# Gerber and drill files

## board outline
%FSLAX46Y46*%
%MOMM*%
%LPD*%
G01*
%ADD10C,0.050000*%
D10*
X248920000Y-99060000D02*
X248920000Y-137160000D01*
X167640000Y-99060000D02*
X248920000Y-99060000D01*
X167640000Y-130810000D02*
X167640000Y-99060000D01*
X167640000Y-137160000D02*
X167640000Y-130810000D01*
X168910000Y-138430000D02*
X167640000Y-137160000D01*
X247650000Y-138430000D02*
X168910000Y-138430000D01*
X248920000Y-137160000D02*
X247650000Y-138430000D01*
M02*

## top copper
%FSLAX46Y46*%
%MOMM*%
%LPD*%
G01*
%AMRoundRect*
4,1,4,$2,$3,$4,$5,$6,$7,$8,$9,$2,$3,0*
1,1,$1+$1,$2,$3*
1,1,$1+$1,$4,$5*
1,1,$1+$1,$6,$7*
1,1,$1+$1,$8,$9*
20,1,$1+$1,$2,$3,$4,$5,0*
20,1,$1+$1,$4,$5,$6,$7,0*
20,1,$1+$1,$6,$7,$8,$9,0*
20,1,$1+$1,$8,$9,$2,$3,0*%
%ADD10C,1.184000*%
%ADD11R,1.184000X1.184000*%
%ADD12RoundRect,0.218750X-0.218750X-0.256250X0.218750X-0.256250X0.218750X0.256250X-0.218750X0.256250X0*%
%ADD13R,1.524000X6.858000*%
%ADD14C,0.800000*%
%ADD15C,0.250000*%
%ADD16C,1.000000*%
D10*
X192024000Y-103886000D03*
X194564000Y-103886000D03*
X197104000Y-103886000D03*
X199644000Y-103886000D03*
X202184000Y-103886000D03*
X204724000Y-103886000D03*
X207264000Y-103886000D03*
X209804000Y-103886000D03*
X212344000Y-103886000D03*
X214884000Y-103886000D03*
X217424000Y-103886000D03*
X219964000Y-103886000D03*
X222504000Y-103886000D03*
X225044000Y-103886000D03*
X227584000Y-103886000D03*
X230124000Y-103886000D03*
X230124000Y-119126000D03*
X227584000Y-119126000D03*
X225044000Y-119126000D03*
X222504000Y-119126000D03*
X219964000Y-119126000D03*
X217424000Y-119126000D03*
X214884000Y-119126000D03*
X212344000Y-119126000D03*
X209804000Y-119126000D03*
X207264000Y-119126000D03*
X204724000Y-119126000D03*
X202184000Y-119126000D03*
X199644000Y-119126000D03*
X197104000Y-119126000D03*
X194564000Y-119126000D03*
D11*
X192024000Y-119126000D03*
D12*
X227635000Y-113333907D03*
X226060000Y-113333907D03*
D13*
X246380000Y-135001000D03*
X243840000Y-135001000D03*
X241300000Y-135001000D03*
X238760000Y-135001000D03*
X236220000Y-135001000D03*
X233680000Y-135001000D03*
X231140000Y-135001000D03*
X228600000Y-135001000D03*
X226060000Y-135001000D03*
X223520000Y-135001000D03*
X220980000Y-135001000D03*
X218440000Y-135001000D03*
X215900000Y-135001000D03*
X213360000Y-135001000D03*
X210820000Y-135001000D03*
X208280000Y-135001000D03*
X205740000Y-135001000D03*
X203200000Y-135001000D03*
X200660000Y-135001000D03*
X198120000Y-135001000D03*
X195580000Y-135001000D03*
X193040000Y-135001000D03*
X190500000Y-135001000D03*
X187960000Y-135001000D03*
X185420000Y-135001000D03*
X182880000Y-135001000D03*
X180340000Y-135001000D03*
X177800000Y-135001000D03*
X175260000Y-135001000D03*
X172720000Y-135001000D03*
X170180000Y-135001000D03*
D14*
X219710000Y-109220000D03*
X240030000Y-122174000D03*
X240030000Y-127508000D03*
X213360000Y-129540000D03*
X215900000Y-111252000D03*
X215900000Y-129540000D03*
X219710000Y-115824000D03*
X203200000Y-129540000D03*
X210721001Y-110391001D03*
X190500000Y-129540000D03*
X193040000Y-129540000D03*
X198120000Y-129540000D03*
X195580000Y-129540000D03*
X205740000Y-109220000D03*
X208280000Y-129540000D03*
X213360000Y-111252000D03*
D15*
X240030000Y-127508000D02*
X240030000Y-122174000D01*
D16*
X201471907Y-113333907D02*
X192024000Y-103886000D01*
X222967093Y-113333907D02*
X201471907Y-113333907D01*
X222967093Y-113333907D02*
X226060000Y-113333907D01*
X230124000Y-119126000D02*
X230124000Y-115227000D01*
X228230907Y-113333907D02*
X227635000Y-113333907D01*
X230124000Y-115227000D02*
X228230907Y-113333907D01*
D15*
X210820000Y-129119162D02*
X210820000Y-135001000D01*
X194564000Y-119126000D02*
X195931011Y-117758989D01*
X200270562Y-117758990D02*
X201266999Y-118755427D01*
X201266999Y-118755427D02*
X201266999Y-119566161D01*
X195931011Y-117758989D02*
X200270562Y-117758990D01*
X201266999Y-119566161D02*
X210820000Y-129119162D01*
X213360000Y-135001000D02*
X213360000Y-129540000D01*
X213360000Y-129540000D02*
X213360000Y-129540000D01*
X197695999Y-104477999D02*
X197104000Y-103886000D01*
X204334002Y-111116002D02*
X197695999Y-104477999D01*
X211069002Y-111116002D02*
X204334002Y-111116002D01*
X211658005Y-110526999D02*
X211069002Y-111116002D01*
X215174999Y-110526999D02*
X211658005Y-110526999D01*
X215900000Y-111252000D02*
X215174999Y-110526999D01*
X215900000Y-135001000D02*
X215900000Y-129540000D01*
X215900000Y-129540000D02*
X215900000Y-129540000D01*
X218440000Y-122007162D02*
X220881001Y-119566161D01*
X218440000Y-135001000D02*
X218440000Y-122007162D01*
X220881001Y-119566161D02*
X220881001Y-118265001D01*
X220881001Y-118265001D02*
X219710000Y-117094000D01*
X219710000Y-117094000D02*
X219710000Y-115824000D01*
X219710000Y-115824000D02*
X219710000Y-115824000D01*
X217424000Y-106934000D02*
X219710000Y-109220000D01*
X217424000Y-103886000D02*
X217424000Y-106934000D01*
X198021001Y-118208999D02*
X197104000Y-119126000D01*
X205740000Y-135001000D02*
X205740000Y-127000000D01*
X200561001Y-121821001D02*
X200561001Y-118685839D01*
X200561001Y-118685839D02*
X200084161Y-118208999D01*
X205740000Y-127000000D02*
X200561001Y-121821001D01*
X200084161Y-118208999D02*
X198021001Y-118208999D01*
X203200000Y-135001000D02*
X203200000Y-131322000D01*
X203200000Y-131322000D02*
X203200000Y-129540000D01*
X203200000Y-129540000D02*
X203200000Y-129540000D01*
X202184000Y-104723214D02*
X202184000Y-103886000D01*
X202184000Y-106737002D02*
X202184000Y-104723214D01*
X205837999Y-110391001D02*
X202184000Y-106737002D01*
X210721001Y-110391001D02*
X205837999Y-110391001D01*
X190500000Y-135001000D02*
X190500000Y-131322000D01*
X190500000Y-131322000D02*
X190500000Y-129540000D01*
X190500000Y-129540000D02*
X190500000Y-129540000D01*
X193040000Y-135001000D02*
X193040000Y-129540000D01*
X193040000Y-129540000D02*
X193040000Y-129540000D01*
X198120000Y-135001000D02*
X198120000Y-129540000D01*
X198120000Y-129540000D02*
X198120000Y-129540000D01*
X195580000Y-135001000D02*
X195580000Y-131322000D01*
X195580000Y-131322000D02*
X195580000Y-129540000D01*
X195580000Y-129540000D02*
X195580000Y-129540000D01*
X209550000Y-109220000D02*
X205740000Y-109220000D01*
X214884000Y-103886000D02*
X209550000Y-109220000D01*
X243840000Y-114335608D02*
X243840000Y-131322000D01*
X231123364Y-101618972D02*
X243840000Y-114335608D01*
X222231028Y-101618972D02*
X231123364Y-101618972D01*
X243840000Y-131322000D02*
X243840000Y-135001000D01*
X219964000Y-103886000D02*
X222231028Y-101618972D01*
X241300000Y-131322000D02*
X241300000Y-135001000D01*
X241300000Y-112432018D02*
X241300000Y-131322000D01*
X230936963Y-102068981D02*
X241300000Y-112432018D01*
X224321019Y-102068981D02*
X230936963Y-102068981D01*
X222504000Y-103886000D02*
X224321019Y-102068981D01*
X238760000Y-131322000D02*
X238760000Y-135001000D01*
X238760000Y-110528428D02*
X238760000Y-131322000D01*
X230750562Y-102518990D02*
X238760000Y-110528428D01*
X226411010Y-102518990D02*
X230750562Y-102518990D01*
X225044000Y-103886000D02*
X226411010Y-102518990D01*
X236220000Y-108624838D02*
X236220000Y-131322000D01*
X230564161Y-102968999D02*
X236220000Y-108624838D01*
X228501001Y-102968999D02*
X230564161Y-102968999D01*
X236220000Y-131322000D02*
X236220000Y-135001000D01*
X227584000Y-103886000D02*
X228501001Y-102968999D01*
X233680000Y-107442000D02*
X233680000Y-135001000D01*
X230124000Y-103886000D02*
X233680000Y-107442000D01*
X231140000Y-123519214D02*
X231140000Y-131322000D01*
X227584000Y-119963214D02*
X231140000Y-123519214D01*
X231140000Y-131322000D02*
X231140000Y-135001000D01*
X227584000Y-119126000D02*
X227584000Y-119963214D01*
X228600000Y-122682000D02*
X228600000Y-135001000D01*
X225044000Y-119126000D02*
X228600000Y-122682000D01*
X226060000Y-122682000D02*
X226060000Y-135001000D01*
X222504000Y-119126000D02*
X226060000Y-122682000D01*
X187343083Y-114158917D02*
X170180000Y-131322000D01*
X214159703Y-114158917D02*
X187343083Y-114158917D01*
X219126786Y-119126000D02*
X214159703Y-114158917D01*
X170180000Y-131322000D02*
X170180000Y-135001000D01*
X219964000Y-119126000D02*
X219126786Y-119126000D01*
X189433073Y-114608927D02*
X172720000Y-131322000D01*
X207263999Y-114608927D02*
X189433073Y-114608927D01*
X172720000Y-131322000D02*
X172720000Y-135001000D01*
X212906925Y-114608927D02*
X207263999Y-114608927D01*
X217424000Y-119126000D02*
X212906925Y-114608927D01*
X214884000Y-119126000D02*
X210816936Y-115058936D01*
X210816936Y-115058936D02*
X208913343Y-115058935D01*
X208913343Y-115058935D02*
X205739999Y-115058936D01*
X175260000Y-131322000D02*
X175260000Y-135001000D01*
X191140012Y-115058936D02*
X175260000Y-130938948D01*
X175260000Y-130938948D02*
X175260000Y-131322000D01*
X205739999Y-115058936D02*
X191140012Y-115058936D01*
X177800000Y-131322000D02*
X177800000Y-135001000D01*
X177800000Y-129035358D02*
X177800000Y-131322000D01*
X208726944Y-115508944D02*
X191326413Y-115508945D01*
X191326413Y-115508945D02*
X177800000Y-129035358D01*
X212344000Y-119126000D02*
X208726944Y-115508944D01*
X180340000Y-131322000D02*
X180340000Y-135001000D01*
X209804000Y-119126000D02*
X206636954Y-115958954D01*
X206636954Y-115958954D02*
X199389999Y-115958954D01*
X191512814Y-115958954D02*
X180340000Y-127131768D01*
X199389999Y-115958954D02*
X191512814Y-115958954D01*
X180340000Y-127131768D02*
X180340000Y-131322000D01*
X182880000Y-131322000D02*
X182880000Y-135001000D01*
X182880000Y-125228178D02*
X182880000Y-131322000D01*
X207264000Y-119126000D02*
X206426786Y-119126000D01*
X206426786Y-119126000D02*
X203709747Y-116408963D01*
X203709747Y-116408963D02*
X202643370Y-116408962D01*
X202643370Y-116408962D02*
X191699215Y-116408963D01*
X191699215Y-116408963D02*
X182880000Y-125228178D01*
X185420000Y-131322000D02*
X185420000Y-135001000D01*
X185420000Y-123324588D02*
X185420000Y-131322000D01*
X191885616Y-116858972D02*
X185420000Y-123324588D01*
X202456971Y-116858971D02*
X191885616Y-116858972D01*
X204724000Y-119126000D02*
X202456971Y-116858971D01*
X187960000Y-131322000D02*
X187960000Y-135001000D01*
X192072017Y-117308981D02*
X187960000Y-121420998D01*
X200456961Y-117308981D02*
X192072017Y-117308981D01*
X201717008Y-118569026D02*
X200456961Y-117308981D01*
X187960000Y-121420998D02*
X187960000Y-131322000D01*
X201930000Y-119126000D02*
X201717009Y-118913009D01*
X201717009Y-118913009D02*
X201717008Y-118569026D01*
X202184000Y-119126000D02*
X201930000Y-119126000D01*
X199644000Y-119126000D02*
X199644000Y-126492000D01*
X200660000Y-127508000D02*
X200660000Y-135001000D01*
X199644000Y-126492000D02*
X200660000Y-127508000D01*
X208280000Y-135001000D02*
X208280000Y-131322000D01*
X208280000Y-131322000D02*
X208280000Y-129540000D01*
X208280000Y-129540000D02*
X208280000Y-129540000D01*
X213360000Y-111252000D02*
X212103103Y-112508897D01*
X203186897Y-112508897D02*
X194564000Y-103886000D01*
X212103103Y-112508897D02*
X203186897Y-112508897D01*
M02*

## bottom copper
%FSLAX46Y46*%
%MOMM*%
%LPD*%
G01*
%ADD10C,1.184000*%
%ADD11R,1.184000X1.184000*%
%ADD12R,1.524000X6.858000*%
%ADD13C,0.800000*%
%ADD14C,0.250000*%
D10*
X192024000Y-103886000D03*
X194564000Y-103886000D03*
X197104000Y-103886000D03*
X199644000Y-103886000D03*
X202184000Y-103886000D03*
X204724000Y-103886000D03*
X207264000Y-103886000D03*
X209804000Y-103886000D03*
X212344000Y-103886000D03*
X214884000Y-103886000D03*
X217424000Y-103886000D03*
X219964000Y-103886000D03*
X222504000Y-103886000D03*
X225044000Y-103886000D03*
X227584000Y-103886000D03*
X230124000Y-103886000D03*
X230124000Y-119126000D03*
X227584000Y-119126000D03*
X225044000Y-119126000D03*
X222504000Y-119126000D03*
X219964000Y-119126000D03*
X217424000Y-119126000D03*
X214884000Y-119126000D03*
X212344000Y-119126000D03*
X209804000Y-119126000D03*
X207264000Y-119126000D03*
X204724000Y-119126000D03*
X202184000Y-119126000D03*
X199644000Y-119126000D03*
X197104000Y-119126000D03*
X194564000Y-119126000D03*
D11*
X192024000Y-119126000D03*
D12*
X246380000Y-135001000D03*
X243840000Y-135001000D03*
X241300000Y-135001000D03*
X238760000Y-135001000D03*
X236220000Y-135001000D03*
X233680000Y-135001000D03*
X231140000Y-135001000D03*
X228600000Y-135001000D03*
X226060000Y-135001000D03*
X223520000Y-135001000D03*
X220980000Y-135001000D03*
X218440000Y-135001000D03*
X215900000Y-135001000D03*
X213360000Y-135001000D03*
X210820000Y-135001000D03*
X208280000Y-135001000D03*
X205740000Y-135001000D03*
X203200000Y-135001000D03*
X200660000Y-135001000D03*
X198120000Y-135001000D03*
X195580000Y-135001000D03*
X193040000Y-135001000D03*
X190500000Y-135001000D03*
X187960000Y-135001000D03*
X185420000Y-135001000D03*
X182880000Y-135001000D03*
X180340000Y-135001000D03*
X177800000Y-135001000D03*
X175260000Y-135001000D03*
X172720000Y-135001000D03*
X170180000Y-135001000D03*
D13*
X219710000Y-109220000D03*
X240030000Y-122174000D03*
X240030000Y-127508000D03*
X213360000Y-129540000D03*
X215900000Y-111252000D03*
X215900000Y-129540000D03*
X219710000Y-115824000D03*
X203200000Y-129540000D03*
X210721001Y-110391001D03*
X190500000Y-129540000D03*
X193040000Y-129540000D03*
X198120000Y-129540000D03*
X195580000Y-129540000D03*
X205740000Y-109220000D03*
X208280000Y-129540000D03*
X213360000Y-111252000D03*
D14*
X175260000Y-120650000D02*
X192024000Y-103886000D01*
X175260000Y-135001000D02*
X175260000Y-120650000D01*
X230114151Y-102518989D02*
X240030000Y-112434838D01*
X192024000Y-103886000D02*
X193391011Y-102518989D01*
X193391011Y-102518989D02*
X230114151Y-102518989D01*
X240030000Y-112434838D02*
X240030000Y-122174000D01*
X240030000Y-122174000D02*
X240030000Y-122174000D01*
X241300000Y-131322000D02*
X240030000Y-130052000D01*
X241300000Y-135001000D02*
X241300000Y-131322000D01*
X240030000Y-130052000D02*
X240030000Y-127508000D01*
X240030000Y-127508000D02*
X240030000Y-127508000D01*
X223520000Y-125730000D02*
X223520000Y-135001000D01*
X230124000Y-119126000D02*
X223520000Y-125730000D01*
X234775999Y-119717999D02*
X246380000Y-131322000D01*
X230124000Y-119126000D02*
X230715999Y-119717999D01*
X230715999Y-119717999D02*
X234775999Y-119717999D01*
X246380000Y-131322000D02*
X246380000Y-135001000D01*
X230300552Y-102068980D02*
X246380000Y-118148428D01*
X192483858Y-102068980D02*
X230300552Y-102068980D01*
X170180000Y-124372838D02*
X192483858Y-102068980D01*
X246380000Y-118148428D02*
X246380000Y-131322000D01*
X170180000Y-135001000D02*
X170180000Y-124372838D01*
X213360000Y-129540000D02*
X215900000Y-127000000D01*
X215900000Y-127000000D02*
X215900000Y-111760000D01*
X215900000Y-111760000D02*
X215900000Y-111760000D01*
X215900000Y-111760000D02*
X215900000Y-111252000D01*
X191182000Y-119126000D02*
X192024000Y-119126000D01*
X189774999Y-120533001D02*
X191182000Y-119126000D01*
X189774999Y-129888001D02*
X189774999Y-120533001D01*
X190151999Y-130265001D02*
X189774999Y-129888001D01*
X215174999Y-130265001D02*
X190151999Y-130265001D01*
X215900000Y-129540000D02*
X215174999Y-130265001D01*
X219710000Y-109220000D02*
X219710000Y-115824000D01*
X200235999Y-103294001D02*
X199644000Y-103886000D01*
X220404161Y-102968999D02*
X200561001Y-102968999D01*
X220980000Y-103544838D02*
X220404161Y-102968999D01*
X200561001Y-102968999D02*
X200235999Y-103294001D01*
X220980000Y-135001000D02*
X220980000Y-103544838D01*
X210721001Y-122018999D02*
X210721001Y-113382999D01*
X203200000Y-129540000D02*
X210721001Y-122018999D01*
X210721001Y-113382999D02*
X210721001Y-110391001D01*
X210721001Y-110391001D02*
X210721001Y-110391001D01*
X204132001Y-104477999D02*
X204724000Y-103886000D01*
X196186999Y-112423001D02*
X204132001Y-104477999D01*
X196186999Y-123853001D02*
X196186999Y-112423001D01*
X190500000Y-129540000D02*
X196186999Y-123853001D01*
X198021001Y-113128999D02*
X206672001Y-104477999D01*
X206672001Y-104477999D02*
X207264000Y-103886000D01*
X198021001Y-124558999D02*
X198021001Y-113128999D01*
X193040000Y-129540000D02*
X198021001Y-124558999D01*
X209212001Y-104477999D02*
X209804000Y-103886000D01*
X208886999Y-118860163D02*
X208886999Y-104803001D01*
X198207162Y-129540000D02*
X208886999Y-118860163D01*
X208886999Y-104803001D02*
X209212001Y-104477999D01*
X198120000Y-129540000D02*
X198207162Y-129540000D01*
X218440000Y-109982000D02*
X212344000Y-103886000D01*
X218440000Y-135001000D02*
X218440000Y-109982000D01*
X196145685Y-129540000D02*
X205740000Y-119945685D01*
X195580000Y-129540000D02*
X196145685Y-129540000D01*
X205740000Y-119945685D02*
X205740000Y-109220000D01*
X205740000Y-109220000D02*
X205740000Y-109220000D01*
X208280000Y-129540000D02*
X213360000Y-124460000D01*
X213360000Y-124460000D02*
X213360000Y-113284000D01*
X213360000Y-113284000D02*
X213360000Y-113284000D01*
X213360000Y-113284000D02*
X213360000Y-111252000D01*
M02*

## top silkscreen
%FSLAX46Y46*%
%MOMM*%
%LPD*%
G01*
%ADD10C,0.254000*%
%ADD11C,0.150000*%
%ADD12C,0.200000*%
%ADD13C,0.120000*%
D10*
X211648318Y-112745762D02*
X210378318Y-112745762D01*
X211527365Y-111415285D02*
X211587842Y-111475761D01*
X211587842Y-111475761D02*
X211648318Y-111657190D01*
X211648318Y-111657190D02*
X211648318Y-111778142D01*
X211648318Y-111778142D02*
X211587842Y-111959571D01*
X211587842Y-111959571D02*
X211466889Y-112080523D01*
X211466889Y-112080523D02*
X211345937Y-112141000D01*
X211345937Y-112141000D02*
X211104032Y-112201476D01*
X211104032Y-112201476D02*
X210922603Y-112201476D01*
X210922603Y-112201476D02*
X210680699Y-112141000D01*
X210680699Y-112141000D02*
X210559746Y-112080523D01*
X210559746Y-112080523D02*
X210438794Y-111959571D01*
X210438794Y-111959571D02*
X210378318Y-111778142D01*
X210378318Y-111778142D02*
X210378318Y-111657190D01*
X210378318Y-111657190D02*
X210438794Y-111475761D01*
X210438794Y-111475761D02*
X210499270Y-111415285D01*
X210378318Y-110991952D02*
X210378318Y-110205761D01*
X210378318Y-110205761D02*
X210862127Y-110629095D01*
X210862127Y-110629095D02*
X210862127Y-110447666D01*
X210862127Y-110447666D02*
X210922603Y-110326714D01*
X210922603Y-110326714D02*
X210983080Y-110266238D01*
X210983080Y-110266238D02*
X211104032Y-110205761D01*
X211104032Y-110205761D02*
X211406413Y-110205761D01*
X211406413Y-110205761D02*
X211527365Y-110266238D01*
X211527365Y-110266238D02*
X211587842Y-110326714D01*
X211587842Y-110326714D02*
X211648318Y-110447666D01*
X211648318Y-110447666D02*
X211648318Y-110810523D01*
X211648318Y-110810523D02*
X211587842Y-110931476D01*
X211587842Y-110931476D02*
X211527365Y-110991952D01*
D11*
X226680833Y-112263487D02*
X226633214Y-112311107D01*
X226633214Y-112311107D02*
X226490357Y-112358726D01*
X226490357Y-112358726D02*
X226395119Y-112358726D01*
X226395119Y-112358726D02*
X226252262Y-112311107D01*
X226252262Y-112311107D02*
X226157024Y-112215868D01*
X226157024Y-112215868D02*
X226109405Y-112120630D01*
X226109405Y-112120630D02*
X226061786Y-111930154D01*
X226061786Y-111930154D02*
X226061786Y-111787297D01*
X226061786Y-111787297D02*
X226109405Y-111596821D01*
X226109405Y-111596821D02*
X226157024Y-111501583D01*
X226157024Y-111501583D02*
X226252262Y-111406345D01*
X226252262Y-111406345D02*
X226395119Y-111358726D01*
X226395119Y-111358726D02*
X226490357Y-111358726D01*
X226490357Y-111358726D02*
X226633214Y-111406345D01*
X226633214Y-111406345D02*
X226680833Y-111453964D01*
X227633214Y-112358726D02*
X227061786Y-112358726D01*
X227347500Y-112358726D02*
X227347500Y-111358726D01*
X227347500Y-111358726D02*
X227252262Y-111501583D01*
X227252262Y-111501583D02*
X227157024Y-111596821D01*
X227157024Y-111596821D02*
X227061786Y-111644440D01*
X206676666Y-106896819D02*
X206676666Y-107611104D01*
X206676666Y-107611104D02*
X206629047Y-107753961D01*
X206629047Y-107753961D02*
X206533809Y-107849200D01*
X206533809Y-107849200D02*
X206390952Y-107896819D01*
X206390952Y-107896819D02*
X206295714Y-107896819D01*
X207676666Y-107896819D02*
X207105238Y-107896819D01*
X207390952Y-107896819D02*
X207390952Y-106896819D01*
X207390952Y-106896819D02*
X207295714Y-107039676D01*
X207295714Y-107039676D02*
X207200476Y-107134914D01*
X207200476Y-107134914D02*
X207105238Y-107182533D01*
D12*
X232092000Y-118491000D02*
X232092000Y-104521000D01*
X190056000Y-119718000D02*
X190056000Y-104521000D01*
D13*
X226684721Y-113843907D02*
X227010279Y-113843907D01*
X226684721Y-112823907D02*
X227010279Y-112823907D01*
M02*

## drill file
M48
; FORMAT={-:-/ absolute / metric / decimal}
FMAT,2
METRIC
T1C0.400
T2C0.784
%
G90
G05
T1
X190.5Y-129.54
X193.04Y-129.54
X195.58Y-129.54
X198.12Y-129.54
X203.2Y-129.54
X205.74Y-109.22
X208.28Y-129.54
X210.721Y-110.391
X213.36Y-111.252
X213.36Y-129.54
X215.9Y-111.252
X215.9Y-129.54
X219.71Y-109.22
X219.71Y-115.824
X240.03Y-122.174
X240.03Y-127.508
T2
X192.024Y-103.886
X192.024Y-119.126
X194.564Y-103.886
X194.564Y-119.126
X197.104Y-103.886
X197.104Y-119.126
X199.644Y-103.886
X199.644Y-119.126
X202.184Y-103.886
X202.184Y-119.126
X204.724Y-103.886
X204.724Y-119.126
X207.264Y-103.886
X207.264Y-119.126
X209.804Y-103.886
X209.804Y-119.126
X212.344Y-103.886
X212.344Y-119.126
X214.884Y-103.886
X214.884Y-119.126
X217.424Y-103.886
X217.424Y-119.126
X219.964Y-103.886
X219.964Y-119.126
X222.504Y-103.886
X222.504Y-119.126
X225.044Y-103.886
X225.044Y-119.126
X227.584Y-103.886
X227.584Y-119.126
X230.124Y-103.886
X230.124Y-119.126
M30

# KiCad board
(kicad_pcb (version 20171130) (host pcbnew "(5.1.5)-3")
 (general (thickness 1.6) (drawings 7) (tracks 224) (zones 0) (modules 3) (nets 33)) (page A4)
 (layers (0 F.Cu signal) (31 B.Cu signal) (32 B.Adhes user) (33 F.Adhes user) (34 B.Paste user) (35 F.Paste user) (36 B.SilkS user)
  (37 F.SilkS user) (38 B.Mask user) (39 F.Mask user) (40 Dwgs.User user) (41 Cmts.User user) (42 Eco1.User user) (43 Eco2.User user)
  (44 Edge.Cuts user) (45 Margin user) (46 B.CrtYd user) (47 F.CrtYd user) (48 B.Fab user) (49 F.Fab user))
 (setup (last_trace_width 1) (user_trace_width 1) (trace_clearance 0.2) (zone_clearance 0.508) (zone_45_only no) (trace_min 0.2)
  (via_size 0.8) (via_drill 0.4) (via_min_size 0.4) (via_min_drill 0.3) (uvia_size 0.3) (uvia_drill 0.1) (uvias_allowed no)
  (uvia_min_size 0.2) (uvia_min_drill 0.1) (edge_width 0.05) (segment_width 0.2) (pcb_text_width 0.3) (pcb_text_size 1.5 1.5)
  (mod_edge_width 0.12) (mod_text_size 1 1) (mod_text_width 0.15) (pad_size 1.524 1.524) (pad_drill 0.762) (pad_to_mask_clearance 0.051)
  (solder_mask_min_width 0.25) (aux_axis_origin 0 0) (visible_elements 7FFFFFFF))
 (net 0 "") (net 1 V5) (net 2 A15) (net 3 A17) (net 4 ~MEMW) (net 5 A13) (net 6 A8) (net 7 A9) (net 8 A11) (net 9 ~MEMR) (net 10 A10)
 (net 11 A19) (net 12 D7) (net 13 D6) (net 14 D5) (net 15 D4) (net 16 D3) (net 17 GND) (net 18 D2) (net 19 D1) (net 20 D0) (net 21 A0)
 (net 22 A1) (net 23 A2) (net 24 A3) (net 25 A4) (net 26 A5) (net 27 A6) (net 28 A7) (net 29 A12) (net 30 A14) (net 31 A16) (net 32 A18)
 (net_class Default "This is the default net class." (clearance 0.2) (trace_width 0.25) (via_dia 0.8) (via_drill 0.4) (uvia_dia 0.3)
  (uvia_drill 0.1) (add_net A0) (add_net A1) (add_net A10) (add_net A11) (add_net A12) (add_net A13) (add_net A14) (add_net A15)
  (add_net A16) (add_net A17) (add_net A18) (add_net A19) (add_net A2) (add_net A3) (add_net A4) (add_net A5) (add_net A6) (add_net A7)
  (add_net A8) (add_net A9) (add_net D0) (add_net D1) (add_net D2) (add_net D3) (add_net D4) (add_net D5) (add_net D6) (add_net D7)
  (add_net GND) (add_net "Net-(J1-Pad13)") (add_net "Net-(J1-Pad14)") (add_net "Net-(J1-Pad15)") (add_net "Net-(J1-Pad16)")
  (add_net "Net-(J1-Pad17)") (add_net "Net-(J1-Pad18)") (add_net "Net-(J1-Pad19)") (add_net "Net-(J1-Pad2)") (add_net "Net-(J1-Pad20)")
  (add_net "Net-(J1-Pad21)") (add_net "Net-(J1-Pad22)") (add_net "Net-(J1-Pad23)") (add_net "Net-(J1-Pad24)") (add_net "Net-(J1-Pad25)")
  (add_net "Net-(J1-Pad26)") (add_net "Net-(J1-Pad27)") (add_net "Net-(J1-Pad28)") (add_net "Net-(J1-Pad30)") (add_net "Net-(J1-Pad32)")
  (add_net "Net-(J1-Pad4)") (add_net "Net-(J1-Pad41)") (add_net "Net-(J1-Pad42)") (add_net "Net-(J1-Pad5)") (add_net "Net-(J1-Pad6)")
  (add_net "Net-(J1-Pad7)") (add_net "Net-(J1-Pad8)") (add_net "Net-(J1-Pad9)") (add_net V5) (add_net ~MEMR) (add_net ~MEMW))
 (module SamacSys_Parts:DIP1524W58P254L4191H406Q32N (layer F.Cu) (at 211.074 111.506 90)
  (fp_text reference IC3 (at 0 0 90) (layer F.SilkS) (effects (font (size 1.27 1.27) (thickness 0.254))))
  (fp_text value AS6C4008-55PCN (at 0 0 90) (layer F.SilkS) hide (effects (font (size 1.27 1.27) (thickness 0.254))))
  (fp_line (start -6.985 21.018) (end 6.985 21.018) (layer F.SilkS) (width 0.2))
  (fp_line (start -8.212 -21.018) (end 6.985 -21.018) (layer F.SilkS) (width 0.2))
  (pad 32 thru_hole circle (at 7.62 -19.05 90) (size 1.184 1.184) (drill 0.784) (layers *.Cu *.Mask) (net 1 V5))
  (pad 31 thru_hole circle (at 7.62 -16.51 90) (size 1.184 1.184) (drill 0.784) (layers *.Cu *.Mask) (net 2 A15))
  (pad 30 thru_hole circle (at 7.62 -13.97 90) (size 1.184 1.184) (drill 0.784) (layers *.Cu *.Mask) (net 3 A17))
  (pad 29 thru_hole circle (at 7.62 -11.43 90) (size 1.184 1.184) (drill 0.784) (layers *.Cu *.Mask) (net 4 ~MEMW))
  (pad 28 thru_hole circle (at 7.62 -8.89 90) (size 1.184 1.184) (drill 0.784) (layers *.Cu *.Mask) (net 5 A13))
  (pad 27 thru_hole circle (at 7.62 -6.35 90) (size 1.184 1.184) (drill 0.784) (layers *.Cu *.Mask) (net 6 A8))
  (pad 26 thru_hole circle (at 7.62 -3.81 90) (size 1.184 1.184) (drill 0.784) (layers *.Cu *.Mask) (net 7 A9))
  (pad 25 thru_hole circle (at 7.62 -1.27 90) (size 1.184 1.184) (drill 0.784) (layers *.Cu *.Mask) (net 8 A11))
  (pad 24 thru_hole circle (at 7.62 1.27 90) (size 1.184 1.184) (drill 0.784) (layers *.Cu *.Mask) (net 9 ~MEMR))
  (pad 23 thru_hole circle (at 7.62 3.81 90) (size 1.184 1.184) (drill 0.784) (layers *.Cu *.Mask) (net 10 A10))
  (pad 22 thru_hole circle (at 7.62 6.35 90) (size 1.184 1.184) (drill 0.784) (layers *.Cu *.Mask) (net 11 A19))
  (pad 21 thru_hole circle (at 7.62 8.89 90) (size 1.184 1.184) (drill 0.784) (layers *.Cu *.Mask) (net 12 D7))
  (pad 20 thru_hole circle (at 7.62 11.43 90) (size 1.184 1.184) (drill 0.784) (layers *.Cu *.Mask) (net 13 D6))
  (pad 19 thru_hole circle (at 7.62 13.97 90) (size 1.184 1.184) (drill 0.784) (layers *.Cu *.Mask) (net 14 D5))
  (pad 18 thru_hole circle (at 7.62 16.51 90) (size 1.184 1.184) (drill 0.784) (layers *.Cu *.Mask) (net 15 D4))
  (pad 17 thru_hole circle (at 7.62 19.05 90) (size 1.184 1.184) (drill 0.784) (layers *.Cu *.Mask) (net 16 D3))
  (pad 16 thru_hole circle (at -7.62 19.05 90) (size 1.184 1.184) (drill 0.784) (layers *.Cu *.Mask) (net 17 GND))
  (pad 15 thru_hole circle (at -7.62 16.51 90) (size 1.184 1.184) (drill 0.784) (layers *.Cu *.Mask) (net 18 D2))
  (pad 14 thru_hole circle (at -7.62 13.97 90) (size 1.184 1.184) (drill 0.784) (layers *.Cu *.Mask) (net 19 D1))
  (pad 13 thru_hole circle (at -7.62 11.43 90) (size 1.184 1.184) (drill 0.784) (layers *.Cu *.Mask) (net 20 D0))
  (pad 12 thru_hole circle (at -7.62 8.89 90) (size 1.184 1.184) (drill 0.784) (layers *.Cu *.Mask) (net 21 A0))
  (pad 11 thru_hole circle (at -7.62 6.35 90) (size 1.184 1.184) (drill 0.784) (layers *.Cu *.Mask) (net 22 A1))
  (pad 10 thru_hole circle (at -7.62 3.81 90) (size 1.184 1.184) (drill 0.784) (layers *.Cu *.Mask) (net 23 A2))
  (pad 9 thru_hole circle (at -7.62 1.27 90) (size 1.184 1.184) (drill 0.784) (layers *.Cu *.Mask) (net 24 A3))
  (pad 8 thru_hole circle (at -7.62 -1.27 90) (size 1.184 1.184) (drill 0.784) (layers *.Cu *.Mask) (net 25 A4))
  (pad 7 thru_hole circle (at -7.62 -3.81 90) (size 1.184 1.184) (drill 0.784) (layers *.Cu *.Mask) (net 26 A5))
  (pad 6 thru_hole circle (at -7.62 -6.35 90) (size 1.184 1.184) (drill 0.784) (layers *.Cu *.Mask) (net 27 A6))
  (pad 5 thru_hole circle (at -7.62 -8.89 90) (size 1.184 1.184) (drill 0.784) (layers *.Cu *.Mask) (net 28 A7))
  (pad 4 thru_hole circle (at -7.62 -11.43 90) (size 1.184 1.184) (drill 0.784) (layers *.Cu *.Mask) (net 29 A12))
  (pad 3 thru_hole circle (at -7.62 -13.97 90) (size 1.184 1.184) (drill 0.784) (layers *.Cu *.Mask) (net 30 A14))
  (pad 2 thru_hole circle (at -7.62 -16.51 90) (size 1.184 1.184) (drill 0.784) (layers *.Cu *.Mask) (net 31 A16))
  (pad 1 thru_hole rect (at -7.62 -19.05 90) (size 1.184 1.184) (drill 0.784) (layers *.Cu *.Mask) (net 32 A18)))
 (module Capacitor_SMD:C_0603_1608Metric (layer F.Cu) (at 226.8475 113.333907)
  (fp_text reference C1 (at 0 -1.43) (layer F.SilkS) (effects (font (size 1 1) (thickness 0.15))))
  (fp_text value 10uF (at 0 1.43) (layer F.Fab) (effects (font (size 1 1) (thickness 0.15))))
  (fp_line (start -0.162779 0.51) (end 0.162779 0.51) (layer F.SilkS) (width 0.12))
  (fp_line (start -0.162779 -0.51) (end 0.162779 -0.51) (layer F.SilkS) (width 0.12))
  (pad 2 smd roundrect (at 0.7875 0) (size 0.875 0.95) (layers F.Cu F.Paste F.Mask) (roundrect_rratio 0.25) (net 17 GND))
  (pad 1 smd roundrect (at -0.7875 0) (size 0.875 0.95) (layers F.Cu F.Paste F.Mask) (roundrect_rratio 0.25) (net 1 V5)))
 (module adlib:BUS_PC (layer F.Cu) (at 208.28 134.62)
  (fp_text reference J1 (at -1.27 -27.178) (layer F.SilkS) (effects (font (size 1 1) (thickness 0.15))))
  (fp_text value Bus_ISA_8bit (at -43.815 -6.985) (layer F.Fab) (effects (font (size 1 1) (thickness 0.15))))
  (pad 1 connect rect (at 38.1 0.381) (size 1.524 6.858) (layers B.Cu B.Mask) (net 17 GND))
  (pad 2 connect rect (at 35.56 0.381) (size 1.524 6.858) (layers B.Cu B.Mask))
  (pad 3 connect rect (at 33.02 0.381) (size 1.524 6.858) (layers B.Cu B.Mask) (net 1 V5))
  (pad 4 connect rect (at 30.48 0.381) (size 1.524 6.858) (layers B.Cu B.Mask))
  (pad 5 connect rect (at 27.94 0.381) (size 1.524 6.858) (layers B.Cu B.Mask))
  (pad 6 connect rect (at 25.4 0.381) (size 1.524 6.858) (layers B.Cu B.Mask))
  (pad 7 connect rect (at 22.86 0.381) (size 1.524 6.858) (layers B.Cu B.Mask))
  (pad 8 connect rect (at 20.32 0.381) (size 1.524 6.858) (layers B.Cu B.Mask))
  (pad 9 connect rect (at 17.78 0.381) (size 1.524 6.858) (layers B.Cu B.Mask))
  (pad 10 connect rect (at 15.24 0.381) (size 1.524 6.858) (layers B.Cu B.Mask) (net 17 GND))
  (pad 11 connect rect (at 12.7 0.381) (size 1.524 6.858) (layers B.Cu B.Mask) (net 4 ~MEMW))
  (pad 12 connect rect (at 10.16 0.381) (size 1.524 6.858) (layers B.Cu B.Mask) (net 9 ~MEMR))
  (pad 13 connect rect (at 7.62 0.381) (size 1.524 6.858) (layers B.Cu B.Mask))
  (pad 14 connect rect (at 5.08 0.381) (size 1.524 6.858) (layers B.Cu B.Mask))
  (pad 15 connect rect (at 2.54 0.381) (size 1.524 6.858) (layers B.Cu B.Mask))
  (pad 16 connect rect (at 0 0.381) (size 1.524 6.858) (layers B.Cu B.Mask))
  (pad 17 connect rect (at -2.54 0.381) (size 1.524 6.858) (layers B.Cu B.Mask))
  (pad 18 connect rect (at -5.08 0.381) (size 1.524 6.858) (layers B.Cu B.Mask))
  (pad 19 connect rect (at -7.62 0.381) (size 1.524 6.858) (layers B.Cu B.Mask))
  (pad 20 connect rect (at -10.16 0.381) (size 1.524 6.858) (layers B.Cu B.Mask))
  (pad 21 connect rect (at -12.7 0.381) (size 1.524 6.858) (layers B.Cu B.Mask))
  (pad 22 connect rect (at -15.24 0.381) (size 1.524 6.858) (layers B.Cu B.Mask))
  (pad 23 connect rect (at -17.78 0.381) (size 1.524 6.858) (layers B.Cu B.Mask))
  (pad 24 connect rect (at -20.32 0.381) (size 1.524 6.858) (layers B.Cu B.Mask))
  (pad 25 connect rect (at -22.86 0.381) (size 1.524 6.858) (layers B.Cu B.Mask))
  (pad 26 connect rect (at -25.4 0.381) (size 1.524 6.858) (layers B.Cu B.Mask))
  (pad 27 connect rect (at -27.94 0.381) (size 1.524 6.858) (layers B.Cu B.Mask))
  (pad 28 connect rect (at -30.48 0.381) (size 1.524 6.858) (layers B.Cu B.Mask))
  (pad 29 connect rect (at -33.02 0.381) (size 1.524 6.858) (layers B.Cu B.Mask) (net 1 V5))
  (pad 30 connect rect (at -35.56 0.381) (size 1.524 6.858) (layers B.Cu B.Mask))
  (pad 31 connect rect (at -38.1 0.381) (size 1.524 6.858) (layers B.Cu B.Mask) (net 17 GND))
  (pad 32 connect rect (at 38.1 0.381) (size 1.524 6.858) (layers F.Cu F.Mask))
  (pad 33 connect rect (at 35.56 0.381) (size 1.524 6.858) (layers F.Cu F.Mask) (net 12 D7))
  (pad 34 connect rect (at 33.02 0.381) (size 1.524 6.858) (layers F.Cu F.Mask) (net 13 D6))
  (pad 35 connect rect (at 30.48 0.381) (size 1.524 6.858) (layers F.Cu F.Mask) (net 14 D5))
  (pad 36 connect rect (at 27.94 0.381) (size 1.524 6.858) (layers F.Cu F.Mask) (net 15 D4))
  (pad 37 connect rect (at 25.4 0.381) (size 1.524 6.858) (layers F.Cu F.Mask) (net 16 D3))
  (pad 38 connect rect (at 22.86 0.381) (size 1.524 6.858) (layers F.Cu F.Mask) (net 18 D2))
  (pad 39 connect rect (at 20.32 0.381) (size 1.524 6.858) (layers F.Cu F.Mask) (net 19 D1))
  (pad 40 connect rect (at 17.78 0.381) (size 1.524 6.858) (layers F.Cu F.Mask) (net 20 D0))
  (pad 41 connect rect (at 15.24 0.381) (size 1.524 6.858) (layers F.Cu F.Mask))
  (pad 42 connect rect (at 12.7 0.381) (size 1.524 6.858) (layers F.Cu F.Mask))
  (pad 43 connect rect (at 10.16 0.381) (size 1.524 6.858) (layers F.Cu F.Mask) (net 11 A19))
  (pad 44 connect rect (at 7.62 0.381) (size 1.524 6.858) (layers F.Cu F.Mask) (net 32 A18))
  (pad 45 connect rect (at 5.08 0.381) (size 1.524 6.858) (layers F.Cu F.Mask) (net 3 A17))
  (pad 46 connect rect (at 2.54 0.381) (size 1.524 6.858) (layers F.Cu F.Mask) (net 31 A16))
  (pad 47 connect rect (at 0 0.381) (size 1.524 6.858) (layers F.Cu F.Mask) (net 2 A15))
  (pad 48 connect rect (at -2.54 0.381) (size 1.524 6.858) (layers F.Cu F.Mask) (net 30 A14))
  (pad 49 connect rect (at -5.08 0.381) (size 1.524 6.858) (layers F.Cu F.Mask) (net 5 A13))
  (pad 50 connect rect (at -7.62 0.381) (size 1.524 6.858) (layers F.Cu F.Mask) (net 29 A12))
  (pad 51 connect rect (at -10.16 0.381) (size 1.524 6.858) (layers F.Cu F.Mask) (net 8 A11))
  (pad 52 connect rect (at -12.7 0.381) (size 1.524 6.858) (layers F.Cu F.Mask) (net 10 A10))
  (pad 53 connect rect (at -15.24 0.381) (size 1.524 6.858) (layers F.Cu F.Mask) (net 7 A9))
  (pad 54 connect rect (at -17.78 0.381) (size 1.524 6.858) (layers F.Cu F.Mask) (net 6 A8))
  (pad 55 connect rect (at -20.32 0.381) (size 1.524 6.858) (layers F.Cu F.Mask) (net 28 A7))
  (pad 56 connect rect (at -22.86 0.381) (size 1.524 6.858) (layers F.Cu F.Mask) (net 27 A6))
  (pad 57 connect rect (at -25.4 0.381) (size 1.524 6.858) (layers F.Cu F.Mask) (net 26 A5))
  (pad 58 connect rect (at -27.94 0.381) (size 1.524 6.858) (layers F.Cu F.Mask) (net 25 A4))
  (pad 59 connect rect (at -30.48 0.381) (size 1.524 6.858) (layers F.Cu F.Mask) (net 24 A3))
  (pad 60 connect rect (at -33.02 0.381) (size 1.524 6.858) (layers F.Cu F.Mask) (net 23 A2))
  (pad 61 connect rect (at -35.56 0.381) (size 1.524 6.858) (layers F.Cu F.Mask) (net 22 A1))
  (pad 62 connect rect (at -38.1 0.381) (size 1.524 6.858) (layers F.Cu F.Mask) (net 21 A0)))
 (gr_line (start 248.92 99.06) (end 248.92 137.16) (layer Edge.Cuts) (width 0.05))
 (gr_line (start 167.64 99.06) (end 248.92 99.06) (layer Edge.Cuts) (width 0.05))
 (gr_line (start 167.64 130.81) (end 167.64 99.06) (layer Edge.Cuts) (width 0.05))
 (gr_line (start 167.64 137.16) (end 167.64 130.81) (layer Edge.Cuts) (width 0.05))
 (gr_line (start 168.91 138.43) (end 167.64 137.16) (layer Edge.Cuts) (width 0.05))
 (gr_line (start 247.65 138.43) (end 168.91 138.43) (layer Edge.Cuts) (width 0.05))
 (gr_line (start 248.92 137.16) (end 247.65 138.43) (layer Edge.Cuts) (width 0.05))
 (via (at 219.71 109.22) (size 0.8) (drill 0.4) (layers F.Cu B.Cu) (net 11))
 (segment (start 175.26 120.65) (end 192.024 103.886) (width 0.25) (layer B.Cu) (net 1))
 (segment (start 175.26 135.001) (end 175.26 120.65) (width 0.25) (layer B.Cu) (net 1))
 (segment (start 230.114151 102.518989) (end 240.03 112.434838) (width 0.25) (layer B.Cu) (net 1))
 (segment (start 192.024 103.886) (end 193.391011 102.518989) (width 0.25) (layer B.Cu) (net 1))
 (segment (start 193.391011 102.518989) (end 230.114151 102.518989) (width 0.25) (layer B.Cu) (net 1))
 (segment (start 240.03 112.434838) (end 240.03 122.174) (width 0.25) (layer B.Cu) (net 1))
 (segment (start 240.03 122.174) (end 240.03 122.174) (width 0.25) (layer B.Cu) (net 1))
 (via (at 240.03 122.174) (size 0.8) (drill 0.4) (layers F.Cu B.Cu) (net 1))
 (segment (start 241.3 131.322) (end 240.03 130.052) (width 0.25) (layer B.Cu) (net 1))
 (segment (start 241.3 135.001) (end 241.3 131.322) (width 0.25) (layer B.Cu) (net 1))
 (segment (start 240.03 130.052) (end 240.03 127.508) (width 0.25) (layer B.Cu) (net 1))
 (segment (start 240.03 127.508) (end 240.03 127.508) (width 0.25) (layer B.Cu) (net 1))
 (via (at 240.03 127.508) (size 0.8) (drill 0.4) (layers F.Cu B.Cu) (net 1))
 (segment (start 240.03 127.508) (end 240.03 122.174) (width 0.25) (layer F.Cu) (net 1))
 (segment (start 201.471907 113.333907) (end 192.024 103.886) (width 1) (layer F.Cu) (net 1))
 (segment (start 222.967093 113.333907) (end 201.471907 113.333907) (width 1) (layer F.Cu) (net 1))
 (segment (start 222.967093 113.333907) (end 226.06 113.333907) (width 1) (layer F.Cu) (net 1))
 (segment (start 223.52 125.73) (end 223.52 135.001) (width 0.25) (layer B.Cu) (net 17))
 (segment (start 230.124 119.126) (end 223.52 125.73) (width 0.25) (layer B.Cu) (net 17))
 (segment (start 234.775999 119.717999) (end 246.38 131.322) (width 0.25) (layer B.Cu) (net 17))
 (segment (start 230.124 119.126) (end 230.715999 119.717999) (width 0.25) (layer B.Cu) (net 17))
 (segment (start 230.715999 119.717999) (end 234.775999 119.717999) (width 0.25) (layer B.Cu) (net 17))
 (segment (start 246.38 131.322) (end 246.38 135.001) (width 0.25) (layer B.Cu) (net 17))
 (segment (start 230.300552 102.06898) (end 246.38 118.148428) (width 0.25) (layer B.Cu) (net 17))
 (segment (start 192.483858 102.06898) (end 230.300552 102.06898) (width 0.25) (layer B.Cu) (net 17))
 (segment (start 170.18 124.372838) (end 192.483858 102.06898) (width 0.25) (layer B.Cu) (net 17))
 (segment (start 246.38 118.148428) (end 246.38 131.322) (width 0.25) (layer B.Cu) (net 17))
 (segment (start 170.18 135.001) (end 170.18 124.372838) (width 0.25) (layer B.Cu) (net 17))
 (segment (start 230.124 119.126) (end 230.124 115.227) (width 1) (layer F.Cu) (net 17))
 (segment (start 228.230907 113.333907) (end 227.635 113.333907) (width 1) (layer F.Cu) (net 17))
 (segment (start 230.124 115.227) (end 228.230907 113.333907) (width 1) (layer F.Cu) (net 17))
 (segment (start 210.82 129.119162) (end 210.82 135.001) (width 0.25) (layer F.Cu) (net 31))
 (segment (start 194.564 119.126) (end 195.931011 117.758989) (width 0.25) (layer F.Cu) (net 31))
 (segment (start 200.270562 117.75899) (end 201.266999 118.755427) (width 0.25) (layer F.Cu) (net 31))
 (segment (start 201.266999 118.755427) (end 201.266999 119.566161) (width 0.25) (layer F.Cu) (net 31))
 (segment (start 195.931011 117.758989) (end 200.270562 117.75899) (width 0.25) (layer F.Cu) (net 31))
 (segment (start 201.266999 119.566161) (end 210.82 129.119162) (width 0.25) (layer F.Cu) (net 31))
 (segment (start 213.36 135.001) (end 213.36 129.54) (width 0.25) (layer F.Cu) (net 3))
 (segment (start 213.36 129.54) (end 213.36 129.54) (width 0.25) (layer F.Cu) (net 3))
 (via (at 213.36 129.54) (size 0.8) (drill 0.4) (layers F.Cu B.Cu) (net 3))
 (segment (start 213.36 129.54) (end 215.9 127) (width 0.25) (layer B.Cu) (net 3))
 (segment (start 215.9 127) (end 215.9 111.76) (width 0.25) (layer B.Cu) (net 3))
 (segment (start 215.9 111.76) (end 215.9 111.76) (width 0.25) (layer B.Cu) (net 3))
 (via (at 215.9 111.252) (size 0.8) (drill 0.4) (layers F.Cu B.Cu) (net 3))
 (segment (start 197.695999 104.477999) (end 197.104 103.886) (width 0.25) (layer F.Cu) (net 3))
 (segment (start 204.334002 111.116002) (end 197.695999 104.477999) (width 0.25) (layer F.Cu) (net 3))
 (segment (start 211.069002 111.116002) (end 204.334002 111.116002) (width 0.25) (layer F.Cu) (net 3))
 (segment (start 211.658005 110.526999) (end 211.069002 111.116002) (width 0.25) (layer F.Cu) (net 3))
 (segment (start 215.174999 110.526999) (end 211.658005 110.526999) (width 0.25) (layer F.Cu) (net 3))
 (segment (start 215.9 111.252) (end 215.174999 110.526999) (width 0.25) (layer F.Cu) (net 3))
 (segment (start 215.9 111.76) (end 215.9 111.252) (width 0.25) (layer B.Cu) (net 3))
 (segment (start 215.9 135.001) (end 215.9 129.54) (width 0.25) (layer F.Cu) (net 32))
 (segment (start 215.9 129.54) (end 215.9 129.54) (width 0.25) (layer F.Cu) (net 32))
 (via (at 215.9 129.54) (size 0.8) (drill 0.4) (layers F.Cu B.Cu) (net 32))
 (segment (start 191.182 119.126) (end 192.024 119.126) (width 0.25) (layer B.Cu) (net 32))
 (segment (start 189.774999 120.533001) (end 191.182 119.126) (width 0.25) (layer B.Cu) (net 32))
 (segment (start 189.774999 129.888001) (end 189.774999 120.533001) (width 0.25) (layer B.Cu) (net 32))
 (segment (start 190.151999 130.265001) (end 189.774999 129.888001) (width 0.25) (layer B.Cu) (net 32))
 (segment (start 215.174999 130.265001) (end 190.151999 130.265001) (width 0.25) (layer B.Cu) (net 32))
 (segment (start 215.9 129.54) (end 215.174999 130.265001) (width 0.25) (layer B.Cu) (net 32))
 (segment (start 218.44 122.007162) (end 220.881001 119.566161) (width 0.25) (layer F.Cu) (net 11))
 (segment (start 218.44 135.001) (end 218.44 122.007162) (width 0.25) (layer F.Cu) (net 11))
 (segment (start 220.881001 119.566161) (end 220.881001 118.265001) (width 0.25) (layer F.Cu) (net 11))
 (segment (start 220.881001 118.265001) (end 219.71 117.094) (width 0.25) (layer F.Cu) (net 11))
 (segment (start 219.71 117.094) (end 219.71 115.824) (width 0.25) (layer F.Cu) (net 11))
 (segment (start 219.71 115.824) (end 219.71 115.824) (width 0.25) (layer F.Cu) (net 11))
 (via (at 219.71 115.824) (size 0.8) (drill 0.4) (layers F.Cu B.Cu) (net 11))
 (segment (start 217.424 106.934) (end 219.71 109.22) (width 0.25) (layer F.Cu) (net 11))
 (segment (start 217.424 103.886) (end 217.424 106.934) (width 0.25) (layer F.Cu) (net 11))
 (segment (start 219.71 109.22) (end 219.71 115.824) (width 0.25) (layer B.Cu) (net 11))
 (segment (start 200.235999 103.294001) (end 199.644 103.886) (width 0.25) (layer B.Cu) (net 4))
 (segment (start 220.404161 102.968999) (end 200.561001 102.968999) (width 0.25) (layer B.Cu) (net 4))
 (segment (start 220.98 103.544838) (end 220.404161 102.968999) (width 0.25) (layer B.Cu) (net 4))
 (segment (start 200.561001 102.968999) (end 200.235999 103.294001) (width 0.25) (layer B.Cu) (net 4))
 (segment (start 220.98 135.001) (end 220.98 103.544838) (width 0.25) (layer B.Cu) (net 4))
 (segment (start 198.021001 118.208999) (end 197.104 119.126) (width 0.25) (layer F.Cu) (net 30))
 (segment (start 205.74 135.001) (end 205.74 127) (width 0.25) (layer F.Cu) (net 30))
 (segment (start 200.561001 121.821001) (end 200.561001 118.685839) (width 0.25) (layer F.Cu) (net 30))
 (segment (start 200.561001 118.685839) (end 200.084161 118.208999) (width 0.25) (layer F.Cu) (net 30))
 (segment (start 205.74 127) (end 200.561001 121.821001) (width 0.25) (layer F.Cu) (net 30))
 (segment (start 200.084161 118.208999) (end 198.021001 118.208999) (width 0.25) (layer F.Cu) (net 30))
 (segment (start 203.2 135.001) (end 203.2 131.322) (width 0.25) (layer F.Cu) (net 5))
 (segment (start 203.2 131.322) (end 203.2 129.54) (width 0.25) (layer F.Cu) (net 5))
 (segment (start 203.2 129.54) (end 203.2 129.54) (width 0.25) (layer F.Cu) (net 5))
 (via (at 203.2 129.54) (size 0.8) (drill 0.4) (layers F.Cu B.Cu) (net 5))
 (segment (start 210.721001 122.018999) (end 210.721001 113.382999) (width 0.25) (layer B.Cu) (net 5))
 (segment (start 203.2 129.54) (end 210.721001 122.018999) (width 0.25) (layer B.Cu) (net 5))
 (segment (start 210.721001 113.382999) (end 210.721001 110.391001) (width 0.25) (layer B.Cu) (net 5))
 (segment (start 210.721001 110.391001) (end 210.721001 110.391001) (width 0.25) (layer B.Cu) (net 5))
 (via (at 210.721001 110.391001) (size 0.8) (drill 0.4) (layers F.Cu B.Cu) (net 5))
 (segment (start 202.184 104.723214) (end 202.184 103.886) (width 0.25) (layer F.Cu) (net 5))
 (segment (start 202.184 106.737002) (end 202.184 104.723214) (width 0.25) (layer F.Cu) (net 5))
 (segment (start 205.837999 110.391001) (end 202.184 106.737002) (width 0.25) (layer F.Cu) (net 5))
 (segment (start 210.721001 110.391001) (end 205.837999 110.391001) (width 0.25) (layer F.Cu) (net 5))
 (segment (start 190.5 135.001) (end 190.5 131.322) (width 0.25) (layer F.Cu) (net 6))
 (segment (start 190.5 131.322) (end 190.5 129.54) (width 0.25) (layer F.Cu) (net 6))
 (segment (start 190.5 129.54) (end 190.5 129.54) (width 0.25) (layer F.Cu) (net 6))
 (via (at 190.5 129.54) (size 0.8) (drill 0.4) (layers F.Cu B.Cu) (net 6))
 (segment (start 204.132001 104.477999) (end 204.724 103.886) (width 0.25) (layer B.Cu) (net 6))
 (segment (start 196.186999 112.423001) (end 204.132001 104.477999) (width 0.25) (layer B.Cu) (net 6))
 (segment (start 196.186999 123.853001) (end 196.186999 112.423001) (width 0.25) (layer B.Cu) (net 6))
 (segment (start 190.5 129.54) (end 196.186999 123.853001) (width 0.25) (layer B.Cu) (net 6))
 (segment (start 193.04 135.001) (end 193.04 129.54) (width 0.25) (layer F.Cu) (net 7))
 (segment (start 193.04 129.54) (end 193.04 129.54) (width 0.25) (layer F.Cu) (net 7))
 (via (at 193.04 129.54) (size 0.8) (drill 0.4) (layers F.Cu B.Cu) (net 7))
 (segment (start 198.021001 113.128999) (end 206.672001 104.477999) (width 0.25) (layer B.Cu) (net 7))
 (segment (start 206.672001 104.477999) (end 207.264 103.886) (width 0.25) (layer B.Cu) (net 7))
 (segment (start 198.021001 124.558999) (end 198.021001 113.128999) (width 0.25) (layer B.Cu) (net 7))
 (segment (start 193.04 129.54) (end 198.021001 124.558999) (width 0.25) (layer B.Cu) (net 7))
 (segment (start 198.12 135.001) (end 198.12 129.54) (width 0.25) (layer F.Cu) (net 8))
 (segment (start 198.12 129.54) (end 198.12 129.54) (width 0.25) (layer F.Cu) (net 8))
 (via (at 198.12 129.54) (size 0.8) (drill 0.4) (layers F.Cu B.Cu) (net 8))
 (segment (start 209.212001 104.477999) (end 209.804 103.886) (width 0.25) (layer B.Cu) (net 8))
 (segment (start 208.886999 118.860163) (end 208.886999 104.803001) (width 0.25) (layer B.Cu) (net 8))
 (segment (start 198.207162 129.54) (end 208.886999 118.860163) (width 0.25) (layer B.Cu) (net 8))
 (segment (start 208.886999 104.803001) (end 209.212001 104.477999) (width 0.25) (layer B.Cu) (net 8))
 (segment (start 198.12 129.54) (end 198.207162 129.54) (width 0.25) (layer B.Cu) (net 8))
 (segment (start 218.44 109.982) (end 212.344 103.886) (width 0.25) (layer B.Cu) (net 9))
 (segment (start 218.44 135.001) (end 218.44 109.982) (width 0.25) (layer B.Cu) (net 9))
 (segment (start 195.58 135.001) (end 195.58 131.322) (width 0.25) (layer F.Cu) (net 10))
 (segment (start 195.58 131.322) (end 195.58 129.54) (width 0.25) (layer F.Cu) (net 10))
 (segment (start 195.58 129.54) (end 195.58 129.54) (width 0.25) (layer F.Cu) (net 10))
 (via (at 195.58 129.54) (size 0.8) (drill 0.4) (layers F.Cu B.Cu) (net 10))
 (segment (start 196.145685 129.54) (end 205.74 119.945685) (width 0.25) (layer B.Cu) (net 10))
 (segment (start 195.58 129.54) (end 196.145685 129.54) (width 0.25) (layer B.Cu) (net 10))
 (segment (start 205.74 119.945685) (end 205.74 109.22) (width 0.25) (layer B.Cu) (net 10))
 (segment (start 205.74 109.22) (end 205.74 109.22) (width 0.25) (layer B.Cu) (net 10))
 (via (at 205.74 109.22) (size 0.8) (drill 0.4) (layers F.Cu B.Cu) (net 10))
 (segment (start 209.55 109.22) (end 205.74 109.22) (width 0.25) (layer F.Cu) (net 10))
 (segment (start 214.884 103.886) (end 209.55 109.22) (width 0.25) (layer F.Cu) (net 10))
 (segment (start 243.84 114.335608) (end 243.84 131.322) (width 0.25) (layer F.Cu) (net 12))
 (segment (start 231.123364 101.618972) (end 243.84 114.335608) (width 0.25) (layer F.Cu) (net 12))
 (segment (start 222.231028 101.618972) (end 231.123364 101.618972) (width 0.25) (layer F.Cu) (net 12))
 (segment (start 243.84 131.322) (end 243.84 135.001) (width 0.25) (layer F.Cu) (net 12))
 (segment (start 219.964 103.886) (end 222.231028 101.618972) (width 0.25) (layer F.Cu) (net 12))
 (segment (start 241.3 131.322) (end 241.3 135.001) (width 0.25) (layer F.Cu) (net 13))
 (segment (start 241.3 112.432018) (end 241.3 131.322) (width 0.25) (layer F.Cu) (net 13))
 (segment (start 230.936963 102.068981) (end 241.3 112.432018) (width 0.25) (layer F.Cu) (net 13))
 (segment (start 224.321019 102.068981) (end 230.936963 102.068981) (width 0.25) (layer F.Cu) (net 13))
 (segment (start 222.504 103.886) (end 224.321019 102.068981) (width 0.25) (layer F.Cu) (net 13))
 (segment (start 238.76 131.322) (end 238.76 135.001) (width 0.25) (layer F.Cu) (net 14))
 (segment (start 238.76 110.528428) (end 238.76 131.322) (width 0.25) (layer F.Cu) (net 14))
 (segment (start 230.750562 102.51899) (end 238.76 110.528428) (width 0.25) (layer F.Cu) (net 14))
 (segment (start 226.41101 102.51899) (end 230.750562 102.51899) (width 0.25) (layer F.Cu) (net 14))
 (segment (start 225.044 103.886) (end 226.41101 102.51899) (width 0.25) (layer F.Cu) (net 14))
 (segment (start 236.22 108.624838) (end 236.22 131.322) (width 0.25) (layer F.Cu) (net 15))
 (segment (start 230.564161 102.968999) (end 236.22 108.624838) (width 0.25) (layer F.Cu) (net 15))
 (segment (start 228.501001 102.968999) (end 230.564161 102.968999) (width 0.25) (layer F.Cu) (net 15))
 (segment (start 236.22 131.322) (end 236.22 135.001) (width 0.25) (layer F.Cu) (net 15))
 (segment (start 227.584 103.886) (end 228.501001 102.968999) (width 0.25) (layer F.Cu) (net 15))
 (segment (start 233.68 107.442) (end 233.68 135.001) (width 0.25) (layer F.Cu) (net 16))
 (segment (start 230.124 103.886) (end 233.68 107.442) (width 0.25) (layer F.Cu) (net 16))
 (segment (start 231.14 123.519214) (end 231.14 131.322) (width 0.25) (layer F.Cu) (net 18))
 (segment (start 227.584 119.963214) (end 231.14 123.519214) (width 0.25) (layer F.Cu) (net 18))
 (segment (start 231.14 131.322) (end 231.14 135.001) (width 0.25) (layer F.Cu) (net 18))
 (segment (start 227.584 119.126) (end 227.584 119.963214) (width 0.25) (layer F.Cu) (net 18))
 (segment (start 228.6 122.682) (end 228.6 135.001) (width 0.25) (layer F.Cu) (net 19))
 (segment (start 225.044 119.126) (end 228.6 122.682) (width 0.25) (layer F.Cu) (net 19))
 (segment (start 226.06 122.682) (end 226.06 135.001) (width 0.25) (layer F.Cu) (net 20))
 (segment (start 222.504 119.126) (end 226.06 122.682) (width 0.25) (layer F.Cu) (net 20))
 (segment (start 187.343083 114.158917) (end 170.18 131.322) (width 0.25) (layer F.Cu) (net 21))
 (segment (start 214.159703 114.158917) (end 187.343083 114.158917) (width 0.25) (layer F.Cu) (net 21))
 (segment (start 219.126786 119.126) (end 214.159703 114.158917) (width 0.25) (layer F.Cu) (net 21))
 (segment (start 170.18 131.322) (end 170.18 135.001) (width 0.25) (layer F.Cu) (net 21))
 (segment (start 219.964 119.126) (end 219.126786 119.126) (width 0.25) (layer F.Cu) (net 21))
 (segment (start 189.433073 114.608927) (end 172.72 131.322) (width 0.25) (layer F.Cu) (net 22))
 (segment (start 207.263999 114.608927) (end 189.433073 114.608927) (width 0.25) (layer F.Cu) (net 22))
 (segment (start 172.72 131.322) (end 172.72 135.001) (width 0.25) (layer F.Cu) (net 22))
 (segment (start 212.906925 114.608927) (end 207.263999 114.608927) (width 0.25) (layer F.Cu) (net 22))
 (segment (start 217.424 119.126) (end 212.906925 114.608927) (width 0.25) (layer F.Cu) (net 22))
 (segment (start 214.884 119.126) (end 210.816936 115.058936) (width 0.25) (layer F.Cu) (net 23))
 (segment (start 210.816936 115.058936) (end 208.913343 115.058935) (width 0.25) (layer F.Cu) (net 23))
 (segment (start 208.913343 115.058935) (end 205.739999 115.058936) (width 0.25) (layer F.Cu) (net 23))
 (segment (start 175.26 131.322) (end 175.26 135.001) (width 0.25) (layer F.Cu) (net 23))
 (segment (start 191.140012 115.058936) (end 175.26 130.938948) (width 0.25) (layer F.Cu) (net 23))
 (segment (start 175.26 130.938948) (end 175.26 131.322) (width 0.25) (layer F.Cu) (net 23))
 (segment (start 205.739999 115.058936) (end 191.140012 115.058936) (width 0.25) (layer F.Cu) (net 23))
 (segment (start 177.8 131.322) (end 177.8 135.001) (width 0.25) (layer F.Cu) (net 24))
 (segment (start 177.8 129.035358) (end 177.8 131.322) (width 0.25) (layer F.Cu) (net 24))
 (segment (start 208.726944 115.508944) (end 191.326413 115.508945) (width 0.25) (layer F.Cu) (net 24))
 (segment (start 191.326413 115.508945) (end 177.8 129.035358) (width 0.25) (layer F.Cu) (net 24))
 (segment (start 212.344 119.126) (end 208.726944 115.508944) (width 0.25) (layer F.Cu) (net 24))
 (segment (start 180.34 131.322) (end 180.34 135.001) (width 0.25) (layer F.Cu) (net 25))
 (segment (start 209.804 119.126) (end 206.636954 115.958954) (width 0.25) (layer F.Cu) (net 25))
 (segment (start 206.636954 115.958954) (end 199.389999 115.958954) (width 0.25) (layer F.Cu) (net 25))
 (segment (start 191.512814 115.958954) (end 180.34 127.131768) (width 0.25) (layer F.Cu) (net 25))
 (segment (start 199.389999 115.958954) (end 191.512814 115.958954) (width 0.25) (layer F.Cu) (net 25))
 (segment (start 180.34 127.131768) (end 180.34 131.322) (width 0.25) (layer F.Cu) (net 25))
 (segment (start 182.88 131.322) (end 182.88 135.001) (width 0.25) (layer F.Cu) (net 26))
 (segment (start 182.88 125.228178) (end 182.88 131.322) (width 0.25) (layer F.Cu) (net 26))
 (segment (start 207.264 119.126) (end 206.426786 119.126) (width 0.25) (layer F.Cu) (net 26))
 (segment (start 206.426786 119.126) (end 203.709747 116.408963) (width 0.25) (layer F.Cu) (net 26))
 (segment (start 203.709747 116.408963) (end 202.64337 116.408962) (width 0.25) (layer F.Cu) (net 26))
 (segment (start 202.64337 116.408962) (end 191.699215 116.408963) (width 0.25) (layer F.Cu) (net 26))
 (segment (start 191.699215 116.408963) (end 182.88 125.228178) (width 0.25) (layer F.Cu) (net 26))
 (segment (start 185.42 131.322) (end 185.42 135.001) (width 0.25) (layer F.Cu) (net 27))
 (segment (start 185.42 123.324588) (end 185.42 131.322) (width 0.25) (layer F.Cu) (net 27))
 (segment (start 191.885616 116.858972) (end 185.42 123.324588) (width 0.25) (layer F.Cu) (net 27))
 (segment (start 202.456971 116.858971) (end 191.885616 116.858972) (width 0.25) (layer F.Cu) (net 27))
 (segment (start 204.724 119.126) (end 202.456971 116.858971) (width 0.25) (layer F.Cu) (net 27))
 (segment (start 187.96 131.322) (end 187.96 135.001) (width 0.25) (layer F.Cu) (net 28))
 (segment (start 192.072017 117.308981) (end 187.96 121.420998) (width 0.25) (layer F.Cu) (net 28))
 (segment (start 200.456961 117.308981) (end 192.072017 117.308981) (width 0.25) (layer F.Cu) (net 28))
 (segment (start 201.717008 118.569026) (end 200.456961 117.308981) (width 0.25) (layer F.Cu) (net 28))
 (segment (start 187.96 121.420998) (end 187.96 131.322) (width 0.25) (layer F.Cu) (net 28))
 (segment (start 201.93 119.126) (end 201.717009 118.913009) (width 0.25) (layer F.Cu) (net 28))
 (segment (start 201.717009 118.913009) (end 201.717008 118.569026) (width 0.25) (layer F.Cu) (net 28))
 (segment (start 202.184 119.126) (end 201.93 119.126) (width 0.25) (layer F.Cu) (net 28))
 (segment (start 199.644 119.126) (end 199.644 126.492) (width 0.25) (layer F.Cu) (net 29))
 (segment (start 200.66 127.508) (end 200.66 135.001) (width 0.25) (layer F.Cu) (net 29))
 (segment (start 199.644 126.492) (end 200.66 127.508) (width 0.25) (layer F.Cu) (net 29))
 (segment (start 208.28 135.001) (end 208.28 131.322) (width 0.25) (layer F.Cu) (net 2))
 (segment (start 208.28 131.322) (end 208.28 129.54) (width 0.25) (layer F.Cu) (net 2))
 (segment (start 208.28 129.54) (end 208.28 129.54) (width 0.25) (layer F.Cu) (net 2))
 (via (at 208.28 129.54) (size 0.8) (drill 0.4) (layers F.Cu B.Cu) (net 2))
 (segment (start 208.28 129.54) (end 213.36 124.46) (width 0.25) (layer B.Cu) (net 2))
 (segment (start 213.36 124.46) (end 213.36 113.284) (width 0.25) (layer B.Cu) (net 2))
 (segment (start 213.36 113.284) (end 213.36 113.284) (width 0.25) (layer B.Cu) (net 2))
 (via (at 213.36 111.252) (size 0.8) (drill 0.4) (layers F.Cu B.Cu) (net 2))
 (segment (start 213.36 113.284) (end 213.36 111.252) (width 0.25) (layer B.Cu) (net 2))
 (segment (start 213.36 111.252) (end 212.103103 112.508897) (width 0.25) (layer F.Cu) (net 2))
 (segment (start 203.186897 112.508897) (end 194.564 103.886) (width 0.25) (layer F.Cu) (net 2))
 (segment (start 212.103103 112.508897) (end 203.186897 112.508897) (width 0.25) (layer F.Cu) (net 2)))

